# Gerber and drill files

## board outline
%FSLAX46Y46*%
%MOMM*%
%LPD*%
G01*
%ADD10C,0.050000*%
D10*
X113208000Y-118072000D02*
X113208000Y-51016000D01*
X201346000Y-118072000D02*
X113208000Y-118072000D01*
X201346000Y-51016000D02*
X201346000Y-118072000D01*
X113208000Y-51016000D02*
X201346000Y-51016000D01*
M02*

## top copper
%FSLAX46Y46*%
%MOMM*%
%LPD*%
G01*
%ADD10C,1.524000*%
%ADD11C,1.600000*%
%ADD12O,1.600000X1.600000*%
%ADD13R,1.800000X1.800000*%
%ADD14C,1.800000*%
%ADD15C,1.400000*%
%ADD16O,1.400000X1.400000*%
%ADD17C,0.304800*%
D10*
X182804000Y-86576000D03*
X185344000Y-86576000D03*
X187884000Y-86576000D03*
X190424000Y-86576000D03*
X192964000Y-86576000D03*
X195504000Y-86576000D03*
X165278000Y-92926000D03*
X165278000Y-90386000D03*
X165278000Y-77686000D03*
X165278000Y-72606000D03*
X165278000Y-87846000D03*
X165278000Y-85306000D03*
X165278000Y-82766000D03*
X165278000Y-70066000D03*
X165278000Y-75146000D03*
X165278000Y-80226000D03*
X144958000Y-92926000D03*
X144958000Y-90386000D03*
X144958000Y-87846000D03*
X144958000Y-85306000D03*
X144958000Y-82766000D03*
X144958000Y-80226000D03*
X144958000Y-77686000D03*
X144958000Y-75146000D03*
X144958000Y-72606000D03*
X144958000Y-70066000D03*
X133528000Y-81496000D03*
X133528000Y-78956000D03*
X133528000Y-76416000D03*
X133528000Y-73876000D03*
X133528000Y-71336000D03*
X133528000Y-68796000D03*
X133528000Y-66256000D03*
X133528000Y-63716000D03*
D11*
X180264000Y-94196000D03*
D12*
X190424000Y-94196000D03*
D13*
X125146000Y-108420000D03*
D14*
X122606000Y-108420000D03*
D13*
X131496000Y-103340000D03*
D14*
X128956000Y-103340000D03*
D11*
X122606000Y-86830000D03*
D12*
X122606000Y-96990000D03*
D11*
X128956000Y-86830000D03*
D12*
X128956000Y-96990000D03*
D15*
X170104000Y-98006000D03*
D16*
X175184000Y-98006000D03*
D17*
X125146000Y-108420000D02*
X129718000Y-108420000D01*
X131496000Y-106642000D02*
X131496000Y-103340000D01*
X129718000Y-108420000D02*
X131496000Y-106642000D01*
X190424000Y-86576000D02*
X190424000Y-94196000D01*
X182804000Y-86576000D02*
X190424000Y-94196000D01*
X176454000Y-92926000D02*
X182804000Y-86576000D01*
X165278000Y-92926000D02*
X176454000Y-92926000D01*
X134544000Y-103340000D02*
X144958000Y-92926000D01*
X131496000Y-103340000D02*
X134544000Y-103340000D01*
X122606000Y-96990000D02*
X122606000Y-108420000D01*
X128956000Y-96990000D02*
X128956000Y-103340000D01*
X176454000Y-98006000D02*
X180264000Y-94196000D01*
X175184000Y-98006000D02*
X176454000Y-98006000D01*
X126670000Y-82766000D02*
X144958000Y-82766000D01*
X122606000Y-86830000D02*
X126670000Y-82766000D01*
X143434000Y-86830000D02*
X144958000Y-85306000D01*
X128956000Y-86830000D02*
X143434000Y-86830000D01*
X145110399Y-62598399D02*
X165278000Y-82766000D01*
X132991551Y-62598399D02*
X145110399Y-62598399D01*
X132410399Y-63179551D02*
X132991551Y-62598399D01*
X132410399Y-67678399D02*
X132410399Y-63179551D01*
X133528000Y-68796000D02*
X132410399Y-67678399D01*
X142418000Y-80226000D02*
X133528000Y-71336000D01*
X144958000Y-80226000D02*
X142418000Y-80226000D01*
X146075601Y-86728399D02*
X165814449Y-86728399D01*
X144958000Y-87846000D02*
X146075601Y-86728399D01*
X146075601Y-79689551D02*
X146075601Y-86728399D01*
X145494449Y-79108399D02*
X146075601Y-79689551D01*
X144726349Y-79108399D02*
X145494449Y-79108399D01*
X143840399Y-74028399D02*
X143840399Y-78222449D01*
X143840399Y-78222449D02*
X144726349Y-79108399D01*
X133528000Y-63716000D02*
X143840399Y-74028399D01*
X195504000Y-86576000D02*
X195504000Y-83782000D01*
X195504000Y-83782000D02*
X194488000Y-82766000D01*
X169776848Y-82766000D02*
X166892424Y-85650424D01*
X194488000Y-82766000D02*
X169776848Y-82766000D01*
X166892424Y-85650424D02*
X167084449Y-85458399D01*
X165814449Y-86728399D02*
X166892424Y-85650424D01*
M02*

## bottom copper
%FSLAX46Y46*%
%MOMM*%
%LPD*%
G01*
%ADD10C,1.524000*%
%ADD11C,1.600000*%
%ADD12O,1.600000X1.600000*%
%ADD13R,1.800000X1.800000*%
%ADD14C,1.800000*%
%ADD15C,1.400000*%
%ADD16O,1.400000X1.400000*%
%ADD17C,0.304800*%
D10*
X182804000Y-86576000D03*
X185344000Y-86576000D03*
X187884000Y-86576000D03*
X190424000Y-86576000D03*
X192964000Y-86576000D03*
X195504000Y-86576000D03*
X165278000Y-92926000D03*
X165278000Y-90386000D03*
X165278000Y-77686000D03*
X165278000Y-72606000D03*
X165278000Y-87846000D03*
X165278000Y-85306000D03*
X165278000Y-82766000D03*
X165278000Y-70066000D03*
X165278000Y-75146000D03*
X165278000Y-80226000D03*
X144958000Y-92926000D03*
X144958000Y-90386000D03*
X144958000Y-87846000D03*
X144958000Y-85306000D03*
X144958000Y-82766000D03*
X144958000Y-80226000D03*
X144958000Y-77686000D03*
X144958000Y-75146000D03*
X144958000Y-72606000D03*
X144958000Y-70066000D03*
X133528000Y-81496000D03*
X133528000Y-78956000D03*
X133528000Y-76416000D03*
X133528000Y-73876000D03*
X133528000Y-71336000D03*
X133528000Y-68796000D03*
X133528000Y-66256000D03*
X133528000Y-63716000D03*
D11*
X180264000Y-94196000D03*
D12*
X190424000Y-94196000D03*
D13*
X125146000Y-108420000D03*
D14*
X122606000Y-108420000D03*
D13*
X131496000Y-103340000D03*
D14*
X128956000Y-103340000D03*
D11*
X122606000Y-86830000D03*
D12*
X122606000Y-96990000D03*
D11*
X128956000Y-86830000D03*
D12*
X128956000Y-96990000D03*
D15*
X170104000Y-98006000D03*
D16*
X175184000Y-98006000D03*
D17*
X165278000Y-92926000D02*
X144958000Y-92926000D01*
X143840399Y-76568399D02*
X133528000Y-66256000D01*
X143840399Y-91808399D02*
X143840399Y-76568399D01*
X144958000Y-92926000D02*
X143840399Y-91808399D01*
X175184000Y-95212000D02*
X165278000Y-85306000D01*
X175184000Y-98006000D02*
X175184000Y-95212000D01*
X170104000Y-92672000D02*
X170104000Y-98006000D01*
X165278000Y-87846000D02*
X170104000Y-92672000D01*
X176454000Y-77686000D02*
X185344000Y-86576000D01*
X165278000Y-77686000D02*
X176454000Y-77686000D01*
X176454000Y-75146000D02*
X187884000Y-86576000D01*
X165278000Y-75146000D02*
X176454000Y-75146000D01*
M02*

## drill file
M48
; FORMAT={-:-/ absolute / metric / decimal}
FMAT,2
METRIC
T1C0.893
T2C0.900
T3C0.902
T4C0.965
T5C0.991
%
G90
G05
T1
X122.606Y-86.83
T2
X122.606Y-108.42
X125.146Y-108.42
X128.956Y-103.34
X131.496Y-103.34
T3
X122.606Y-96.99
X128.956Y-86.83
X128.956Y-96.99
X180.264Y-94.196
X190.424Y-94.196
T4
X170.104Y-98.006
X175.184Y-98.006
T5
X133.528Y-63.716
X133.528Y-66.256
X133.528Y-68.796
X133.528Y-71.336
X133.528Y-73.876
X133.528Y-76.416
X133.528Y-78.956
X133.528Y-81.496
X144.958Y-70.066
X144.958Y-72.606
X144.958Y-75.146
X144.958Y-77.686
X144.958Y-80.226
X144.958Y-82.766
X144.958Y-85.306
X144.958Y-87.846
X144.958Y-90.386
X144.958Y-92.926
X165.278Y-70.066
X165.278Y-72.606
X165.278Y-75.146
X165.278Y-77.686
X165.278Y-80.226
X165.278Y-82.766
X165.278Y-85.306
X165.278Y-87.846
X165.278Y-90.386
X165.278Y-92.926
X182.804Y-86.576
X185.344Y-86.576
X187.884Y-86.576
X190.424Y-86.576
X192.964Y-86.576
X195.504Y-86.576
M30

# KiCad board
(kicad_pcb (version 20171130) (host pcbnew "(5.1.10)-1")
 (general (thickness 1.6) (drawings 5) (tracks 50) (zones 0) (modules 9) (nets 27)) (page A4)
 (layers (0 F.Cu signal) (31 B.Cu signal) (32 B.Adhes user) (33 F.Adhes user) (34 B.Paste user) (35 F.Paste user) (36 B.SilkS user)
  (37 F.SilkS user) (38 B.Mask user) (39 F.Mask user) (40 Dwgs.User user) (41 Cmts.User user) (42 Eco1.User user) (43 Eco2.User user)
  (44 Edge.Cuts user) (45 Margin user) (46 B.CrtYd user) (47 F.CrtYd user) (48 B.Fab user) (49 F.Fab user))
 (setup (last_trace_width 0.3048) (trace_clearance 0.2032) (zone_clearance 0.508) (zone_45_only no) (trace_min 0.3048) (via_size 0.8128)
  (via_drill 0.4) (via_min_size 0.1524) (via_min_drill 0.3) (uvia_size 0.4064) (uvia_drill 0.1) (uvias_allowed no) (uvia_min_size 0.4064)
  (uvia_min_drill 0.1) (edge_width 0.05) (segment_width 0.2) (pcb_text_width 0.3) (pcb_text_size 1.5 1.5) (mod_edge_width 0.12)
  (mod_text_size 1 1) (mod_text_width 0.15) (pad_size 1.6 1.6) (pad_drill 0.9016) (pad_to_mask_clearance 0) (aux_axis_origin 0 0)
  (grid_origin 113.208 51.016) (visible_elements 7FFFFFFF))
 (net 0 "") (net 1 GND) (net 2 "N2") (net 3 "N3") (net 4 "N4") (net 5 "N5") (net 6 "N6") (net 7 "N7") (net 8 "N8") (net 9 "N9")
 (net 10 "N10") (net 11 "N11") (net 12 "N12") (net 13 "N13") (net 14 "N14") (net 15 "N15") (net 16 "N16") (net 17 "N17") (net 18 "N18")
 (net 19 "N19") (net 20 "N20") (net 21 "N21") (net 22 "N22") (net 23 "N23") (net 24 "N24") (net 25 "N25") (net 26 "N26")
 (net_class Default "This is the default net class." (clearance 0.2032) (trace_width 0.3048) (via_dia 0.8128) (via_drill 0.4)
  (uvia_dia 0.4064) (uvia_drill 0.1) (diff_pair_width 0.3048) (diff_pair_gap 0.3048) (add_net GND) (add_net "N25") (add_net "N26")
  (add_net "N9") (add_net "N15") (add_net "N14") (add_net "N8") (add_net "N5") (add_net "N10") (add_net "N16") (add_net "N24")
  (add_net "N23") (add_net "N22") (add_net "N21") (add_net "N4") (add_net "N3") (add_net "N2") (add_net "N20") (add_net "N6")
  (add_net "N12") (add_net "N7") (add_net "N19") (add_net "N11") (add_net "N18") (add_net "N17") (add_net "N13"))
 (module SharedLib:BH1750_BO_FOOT (layer F.Cu) (at 189.154 86.576)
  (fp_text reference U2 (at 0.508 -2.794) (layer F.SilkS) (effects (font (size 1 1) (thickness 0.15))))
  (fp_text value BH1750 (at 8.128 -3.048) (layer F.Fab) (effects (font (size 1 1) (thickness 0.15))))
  (pad 6 thru_hole circle (at -6.35 0) (size 1.524 1.524) (drill 0.9906) (layers *.Cu *.Mask) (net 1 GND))
  (pad 5 thru_hole circle (at -3.81 0) (size 1.524 1.524) (drill 0.9906) (layers *.Cu *.Mask) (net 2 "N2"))
  (pad 4 thru_hole circle (at -1.27 0) (size 1.524 1.524) (drill 0.9906) (layers *.Cu *.Mask) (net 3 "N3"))
  (pad 3 thru_hole circle (at 1.27 0) (size 1.524 1.524) (drill 0.9906) (layers *.Cu *.Mask) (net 1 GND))
  (pad 2 thru_hole circle (at 3.81 0) (size 1.524 1.524) (drill 0.9906) (layers *.Cu *.Mask) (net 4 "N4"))
  (pad 1 thru_hole circle (at 6.35 0) (size 1.524 1.524) (drill 0.9906) (layers *.Cu *.Mask) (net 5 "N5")))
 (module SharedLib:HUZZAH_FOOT (layer F.Cu) (at 155.118 81.496)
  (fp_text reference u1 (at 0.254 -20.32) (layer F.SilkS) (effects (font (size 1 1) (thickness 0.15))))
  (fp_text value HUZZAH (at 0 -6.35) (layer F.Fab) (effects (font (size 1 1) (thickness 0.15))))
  (pad 11 thru_hole circle (at 10.16 11.43) (size 1.524 1.524) (drill 0.9906) (layers *.Cu *.Mask) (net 1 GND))
  (pad 12 thru_hole circle (at 10.16 8.89) (size 1.524 1.524) (drill 0.9906) (layers *.Cu *.Mask) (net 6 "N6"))
  (pad 17 thru_hole circle (at 10.16 -3.81) (size 1.524 1.524) (drill 0.9906) (layers *.Cu *.Mask) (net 2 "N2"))
  (pad 19 thru_hole circle (at 10.16 -8.89) (size 1.524 1.524) (drill 0.9906) (layers *.Cu *.Mask) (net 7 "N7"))
  (pad 13 thru_hole circle (at 10.16 6.35) (size 1.524 1.524) (drill 0.9906) (layers *.Cu *.Mask) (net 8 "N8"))
  (pad 14 thru_hole circle (at 10.16 3.81) (size 1.524 1.524) (drill 0.9906) (layers *.Cu *.Mask) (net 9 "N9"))
  (pad 15 thru_hole circle (at 10.16 1.27) (size 1.524 1.524) (drill 0.9906) (layers *.Cu *.Mask) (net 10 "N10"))
  (pad 20 thru_hole circle (at 10.16 -11.43) (size 1.524 1.524) (drill 0.9906) (layers *.Cu *.Mask) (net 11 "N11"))
  (pad 18 thru_hole circle (at 10.16 -6.35) (size 1.524 1.524) (drill 0.9906) (layers *.Cu *.Mask) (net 3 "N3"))
  (pad 16 thru_hole circle (at 10.16 -1.27) (size 1.524 1.524) (drill 0.9906) (layers *.Cu *.Mask) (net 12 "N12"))
  (pad 10 thru_hole circle (at -10.16 11.43) (size 1.524 1.524) (drill 0.9906) (layers *.Cu *.Mask) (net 1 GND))
  (pad 9 thru_hole circle (at -10.16 8.89) (size 1.524 1.524) (drill 0.9906) (layers *.Cu *.Mask) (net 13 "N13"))
  (pad 8 thru_hole circle (at -10.16 6.35) (size 1.524 1.524) (drill 0.9906) (layers *.Cu *.Mask) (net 5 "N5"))
  (pad 7 thru_hole circle (at -10.16 3.81) (size 1.524 1.524) (drill 0.9906) (layers *.Cu *.Mask) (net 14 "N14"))
  (pad 6 thru_hole circle (at -10.16 1.27) (size 1.524 1.524) (drill 0.9906) (layers *.Cu *.Mask) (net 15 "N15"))
  (pad 5 thru_hole circle (at -10.16 -1.27) (size 1.524 1.524) (drill 0.9906) (layers *.Cu *.Mask) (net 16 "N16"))
  (pad 4 thru_hole circle (at -10.16 -3.81) (size 1.524 1.524) (drill 0.9906) (layers *.Cu *.Mask) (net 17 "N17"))
  (pad 3 thru_hole circle (at -10.16 -6.35) (size 1.524 1.524) (drill 0.9906) (layers *.Cu *.Mask) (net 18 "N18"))
  (pad 2 thru_hole circle (at -10.16 -8.89) (size 1.524 1.524) (drill 0.9906) (layers *.Cu *.Mask) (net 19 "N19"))
  (pad 1 thru_hole circle (at -10.16 -11.43) (size 1.524 1.524) (drill 0.9906) (layers *.Cu *.Mask) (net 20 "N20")))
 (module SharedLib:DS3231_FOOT (layer F.Cu) (at 127.178 72.606 90)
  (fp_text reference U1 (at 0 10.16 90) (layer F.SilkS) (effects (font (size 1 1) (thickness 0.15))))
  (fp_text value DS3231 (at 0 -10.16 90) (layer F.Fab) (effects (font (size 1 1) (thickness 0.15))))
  (pad 8 thru_hole circle (at -8.89 6.35 90) (size 1.524 1.524) (drill 0.9906) (layers *.Cu *.Mask) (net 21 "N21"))
  (pad 7 thru_hole circle (at -6.35 6.35 90) (size 1.524 1.524) (drill 0.9906) (layers *.Cu *.Mask) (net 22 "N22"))
  (pad 6 thru_hole circle (at -3.81 6.35 90) (size 1.524 1.524) (drill 0.9906) (layers *.Cu *.Mask) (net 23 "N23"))
  (pad 5 thru_hole circle (at -1.27 6.35 90) (size 1.524 1.524) (drill 0.9906) (layers *.Cu *.Mask) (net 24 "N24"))
  (pad 4 thru_hole circle (at 1.27 6.35 90) (size 1.524 1.524) (drill 0.9906) (layers *.Cu *.Mask) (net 16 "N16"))
  (pad 3 thru_hole circle (at 3.81 6.35 90) (size 1.524 1.524) (drill 0.9906) (layers *.Cu *.Mask) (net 10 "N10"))
  (pad 2 thru_hole circle (at 6.35 6.35 90) (size 1.524 1.524) (drill 0.9906) (layers *.Cu *.Mask) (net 1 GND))
  (pad 1 thru_hole circle (at 8.89 6.35 90) (size 1.524 1.524) (drill 0.9906) (layers *.Cu *.Mask) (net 5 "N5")))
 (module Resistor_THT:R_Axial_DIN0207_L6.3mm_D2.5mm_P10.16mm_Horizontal (layer F.Cu) (at 180.264 94.196)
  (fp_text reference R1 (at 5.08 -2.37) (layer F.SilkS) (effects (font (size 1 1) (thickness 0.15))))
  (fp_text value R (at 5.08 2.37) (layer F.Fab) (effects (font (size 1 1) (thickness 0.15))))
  (pad 1 thru_hole circle (at 0 0) (size 1.6 1.6) (drill 0.9016) (layers *.Cu *.Mask) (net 9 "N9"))
  (pad 2 thru_hole oval (at 10.16 0) (size 1.6 1.6) (drill 0.9016) (layers *.Cu *.Mask) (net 1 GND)))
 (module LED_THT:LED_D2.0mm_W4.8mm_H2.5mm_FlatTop (layer F.Cu) (at 125.146 108.42 180)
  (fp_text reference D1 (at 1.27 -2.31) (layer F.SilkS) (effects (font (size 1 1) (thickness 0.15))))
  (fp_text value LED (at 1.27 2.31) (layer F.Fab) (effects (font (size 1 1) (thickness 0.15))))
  (pad 1 thru_hole rect (at 0 0 180) (size 1.8 1.8) (drill 0.9) (layers *.Cu *.Mask) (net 1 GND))
  (pad 2 thru_hole circle (at 2.54 0 180) (size 1.8 1.8) (drill 0.9) (layers *.Cu *.Mask) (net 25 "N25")))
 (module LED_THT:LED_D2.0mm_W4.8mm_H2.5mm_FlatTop (layer F.Cu) (at 131.496 103.34 180)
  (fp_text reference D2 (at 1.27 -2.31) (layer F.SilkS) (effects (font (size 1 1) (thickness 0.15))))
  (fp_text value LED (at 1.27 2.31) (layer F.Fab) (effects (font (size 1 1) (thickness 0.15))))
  (pad 1 thru_hole rect (at 0 0 180) (size 1.8 1.8) (drill 0.9) (layers *.Cu *.Mask) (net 1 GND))
  (pad 2 thru_hole circle (at 2.54 0 180) (size 1.8 1.8) (drill 0.9) (layers *.Cu *.Mask) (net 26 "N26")))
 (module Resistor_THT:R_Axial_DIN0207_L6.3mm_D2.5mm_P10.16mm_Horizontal (layer F.Cu) (at 122.606 86.83 270)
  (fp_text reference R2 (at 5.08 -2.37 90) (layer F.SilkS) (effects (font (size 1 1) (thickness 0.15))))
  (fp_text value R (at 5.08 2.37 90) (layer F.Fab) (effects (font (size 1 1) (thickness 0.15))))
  (pad 1 thru_hole circle (at 0 0 270) (size 1.6 1.6) (drill 0.8928) (layers *.Cu *.Mask) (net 15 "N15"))
  (pad 2 thru_hole oval (at 10.16 0 270) (size 1.6 1.6) (drill 0.9016) (layers *.Cu *.Mask) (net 25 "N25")))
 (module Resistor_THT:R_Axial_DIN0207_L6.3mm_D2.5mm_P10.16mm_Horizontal (layer F.Cu) (at 128.956 86.83 270)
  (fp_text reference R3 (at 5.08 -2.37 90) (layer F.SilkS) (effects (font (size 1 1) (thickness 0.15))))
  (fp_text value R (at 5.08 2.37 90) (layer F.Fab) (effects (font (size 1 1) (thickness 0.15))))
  (pad 1 thru_hole circle (at 0 0 270) (size 1.6 1.6) (drill 0.9016) (layers *.Cu *.Mask) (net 14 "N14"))
  (pad 2 thru_hole oval (at 10.16 0 270) (size 1.6 1.6) (drill 0.9016) (layers *.Cu *.Mask) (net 26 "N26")))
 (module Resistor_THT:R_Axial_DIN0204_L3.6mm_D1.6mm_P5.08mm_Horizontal (layer F.Cu) (at 170.104 98.006)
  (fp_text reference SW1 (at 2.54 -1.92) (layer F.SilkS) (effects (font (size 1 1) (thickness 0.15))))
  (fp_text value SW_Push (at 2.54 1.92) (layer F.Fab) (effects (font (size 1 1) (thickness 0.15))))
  (pad 1 thru_hole circle (at 0 0) (size 1.4 1.4) (drill 0.9652) (layers *.Cu *.Mask) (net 8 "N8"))
  (pad 2 thru_hole oval (at 5.08 0) (size 1.4 1.4) (drill 0.9652) (layers *.Cu *.Mask B.SilkS) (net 9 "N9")))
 (gr_line (start 113.208 118.072) (end 113.208 51.016) (layer Edge.Cuts) (width 0.05))
 (gr_line (start 201.346 118.072) (end 113.208 118.072) (layer Edge.Cuts) (width 0.05))
 (gr_line (start 201.346 51.016) (end 201.346 118.072) (layer Edge.Cuts) (width 0.05))
 (gr_line (start 113.208 51.016) (end 201.346 51.016) (layer Edge.Cuts) (width 0.05))
 (segment (start 125.146 108.42) (end 129.718 108.42) (width 0.3048) (layer F.Cu) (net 1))
 (segment (start 131.496 106.642) (end 131.496 103.34) (width 0.3048) (layer F.Cu) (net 1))
 (segment (start 129.718 108.42) (end 131.496 106.642) (width 0.3048) (layer F.Cu) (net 1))
 (segment (start 190.424 86.576) (end 190.424 94.196) (width 0.3048) (layer F.Cu) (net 1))
 (segment (start 182.804 86.576) (end 190.424 94.196) (width 0.3048) (layer F.Cu) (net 1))
 (segment (start 176.454 92.926) (end 182.804 86.576) (width 0.3048) (layer F.Cu) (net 1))
 (segment (start 165.278 92.926) (end 176.454 92.926) (width 0.3048) (layer F.Cu) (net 1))
 (segment (start 165.278 92.926) (end 144.958 92.926) (width 0.3048) (layer B.Cu) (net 1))
 (segment (start 134.544 103.34) (end 144.958 92.926) (width 0.3048) (layer F.Cu) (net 1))
 (segment (start 131.496 103.34) (end 134.544 103.34) (width 0.3048) (layer F.Cu) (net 1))
 (segment (start 143.840399 76.568399) (end 133.528 66.256) (width 0.3048) (layer B.Cu) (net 1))
 (segment (start 143.840399 91.808399) (end 143.840399 76.568399) (width 0.3048) (layer B.Cu) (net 1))
 (segment (start 144.958 92.926) (end 143.840399 91.808399) (width 0.3048) (layer B.Cu) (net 1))
 (segment (start 122.606 96.99) (end 122.606 108.42) (width 0.3048) (layer F.Cu) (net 25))
 (segment (start 128.956 96.99) (end 128.956 103.34) (width 0.3048) (layer F.Cu) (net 26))
 (segment (start 176.454 98.006) (end 180.264 94.196) (width 0.3048) (layer F.Cu) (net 9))
 (segment (start 175.184 98.006) (end 176.454 98.006) (width 0.3048) (layer F.Cu) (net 9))
 (segment (start 175.184 95.212) (end 165.278 85.306) (width 0.3048) (layer B.Cu) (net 9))
 (segment (start 175.184 98.006) (end 175.184 95.212) (width 0.3048) (layer B.Cu) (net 9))
 (segment (start 126.67 82.766) (end 144.958 82.766) (width 0.3048) (layer F.Cu) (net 15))
 (segment (start 122.606 86.83) (end 126.67 82.766) (width 0.3048) (layer F.Cu) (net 15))
 (segment (start 143.434 86.83) (end 144.958 85.306) (width 0.3048) (layer F.Cu) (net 14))
 (segment (start 128.956 86.83) (end 143.434 86.83) (width 0.3048) (layer F.Cu) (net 14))
 (segment (start 170.104 92.672) (end 170.104 98.006) (width 0.3048) (layer B.Cu) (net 8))
 (segment (start 165.278 87.846) (end 170.104 92.672) (width 0.3048) (layer B.Cu) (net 8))
 (segment (start 145.110399 62.598399) (end 165.278 82.766) (width 0.3048) (layer F.Cu) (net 10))
 (segment (start 132.991551 62.598399) (end 145.110399 62.598399) (width 0.3048) (layer F.Cu) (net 10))
 (segment (start 132.410399 63.179551) (end 132.991551 62.598399) (width 0.3048) (layer F.Cu) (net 10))
 (segment (start 132.410399 67.678399) (end 132.410399 63.179551) (width 0.3048) (layer F.Cu) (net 10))
 (segment (start 133.528 68.796) (end 132.410399 67.678399) (width 0.3048) (layer F.Cu) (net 10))
 (segment (start 142.418 80.226) (end 133.528 71.336) (width 0.3048) (layer F.Cu) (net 16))
 (segment (start 144.958 80.226) (end 142.418 80.226) (width 0.3048) (layer F.Cu) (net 16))
 (segment (start 176.454 77.686) (end 185.344 86.576) (width 0.3048) (layer B.Cu) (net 2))
 (segment (start 165.278 77.686) (end 176.454 77.686) (width 0.3048) (layer B.Cu) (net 2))
 (segment (start 176.454 75.146) (end 187.884 86.576) (width 0.3048) (layer B.Cu) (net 3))
 (segment (start 165.278 75.146) (end 176.454 75.146) (width 0.3048) (layer B.Cu) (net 3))
 (segment (start 146.075601 86.728399) (end 165.814449 86.728399) (width 0.3048) (layer F.Cu) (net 5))
 (segment (start 144.958 87.846) (end 146.075601 86.728399) (width 0.3048) (layer F.Cu) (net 5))
 (segment (start 146.075601 79.689551) (end 146.075601 86.728399) (width 0.3048) (layer F.Cu) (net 5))
 (segment (start 145.494449 79.108399) (end 146.075601 79.689551) (width 0.3048) (layer F.Cu) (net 5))
 (segment (start 144.726349 79.108399) (end 145.494449 79.108399) (width 0.3048) (layer F.Cu) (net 5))
 (segment (start 143.840399 74.028399) (end 143.840399 78.222449) (width 0.3048) (layer F.Cu) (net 5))
 (segment (start 143.840399 78.222449) (end 144.726349 79.108399) (width 0.3048) (layer F.Cu) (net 5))
 (segment (start 133.528 63.716) (end 143.840399 74.028399) (width 0.3048) (layer F.Cu) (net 5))
 (segment (start 195.504 86.576) (end 195.504 83.782) (width 0.3048) (layer F.Cu) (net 5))
 (segment (start 195.504 83.782) (end 194.488 82.766) (width 0.3048) (layer F.Cu) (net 5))
 (segment (start 169.776848 82.766) (end 166.892424 85.650424) (width 0.3048) (layer F.Cu) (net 5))
 (segment (start 194.488 82.766) (end 169.776848 82.766) (width 0.3048) (layer F.Cu) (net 5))
 (segment (start 166.892424 85.650424) (end 167.084449 85.458399) (width 0.3048) (layer F.Cu) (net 5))
 (segment (start 165.814449 86.728399) (end 166.892424 85.650424) (width 0.3048) (layer F.Cu) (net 5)))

